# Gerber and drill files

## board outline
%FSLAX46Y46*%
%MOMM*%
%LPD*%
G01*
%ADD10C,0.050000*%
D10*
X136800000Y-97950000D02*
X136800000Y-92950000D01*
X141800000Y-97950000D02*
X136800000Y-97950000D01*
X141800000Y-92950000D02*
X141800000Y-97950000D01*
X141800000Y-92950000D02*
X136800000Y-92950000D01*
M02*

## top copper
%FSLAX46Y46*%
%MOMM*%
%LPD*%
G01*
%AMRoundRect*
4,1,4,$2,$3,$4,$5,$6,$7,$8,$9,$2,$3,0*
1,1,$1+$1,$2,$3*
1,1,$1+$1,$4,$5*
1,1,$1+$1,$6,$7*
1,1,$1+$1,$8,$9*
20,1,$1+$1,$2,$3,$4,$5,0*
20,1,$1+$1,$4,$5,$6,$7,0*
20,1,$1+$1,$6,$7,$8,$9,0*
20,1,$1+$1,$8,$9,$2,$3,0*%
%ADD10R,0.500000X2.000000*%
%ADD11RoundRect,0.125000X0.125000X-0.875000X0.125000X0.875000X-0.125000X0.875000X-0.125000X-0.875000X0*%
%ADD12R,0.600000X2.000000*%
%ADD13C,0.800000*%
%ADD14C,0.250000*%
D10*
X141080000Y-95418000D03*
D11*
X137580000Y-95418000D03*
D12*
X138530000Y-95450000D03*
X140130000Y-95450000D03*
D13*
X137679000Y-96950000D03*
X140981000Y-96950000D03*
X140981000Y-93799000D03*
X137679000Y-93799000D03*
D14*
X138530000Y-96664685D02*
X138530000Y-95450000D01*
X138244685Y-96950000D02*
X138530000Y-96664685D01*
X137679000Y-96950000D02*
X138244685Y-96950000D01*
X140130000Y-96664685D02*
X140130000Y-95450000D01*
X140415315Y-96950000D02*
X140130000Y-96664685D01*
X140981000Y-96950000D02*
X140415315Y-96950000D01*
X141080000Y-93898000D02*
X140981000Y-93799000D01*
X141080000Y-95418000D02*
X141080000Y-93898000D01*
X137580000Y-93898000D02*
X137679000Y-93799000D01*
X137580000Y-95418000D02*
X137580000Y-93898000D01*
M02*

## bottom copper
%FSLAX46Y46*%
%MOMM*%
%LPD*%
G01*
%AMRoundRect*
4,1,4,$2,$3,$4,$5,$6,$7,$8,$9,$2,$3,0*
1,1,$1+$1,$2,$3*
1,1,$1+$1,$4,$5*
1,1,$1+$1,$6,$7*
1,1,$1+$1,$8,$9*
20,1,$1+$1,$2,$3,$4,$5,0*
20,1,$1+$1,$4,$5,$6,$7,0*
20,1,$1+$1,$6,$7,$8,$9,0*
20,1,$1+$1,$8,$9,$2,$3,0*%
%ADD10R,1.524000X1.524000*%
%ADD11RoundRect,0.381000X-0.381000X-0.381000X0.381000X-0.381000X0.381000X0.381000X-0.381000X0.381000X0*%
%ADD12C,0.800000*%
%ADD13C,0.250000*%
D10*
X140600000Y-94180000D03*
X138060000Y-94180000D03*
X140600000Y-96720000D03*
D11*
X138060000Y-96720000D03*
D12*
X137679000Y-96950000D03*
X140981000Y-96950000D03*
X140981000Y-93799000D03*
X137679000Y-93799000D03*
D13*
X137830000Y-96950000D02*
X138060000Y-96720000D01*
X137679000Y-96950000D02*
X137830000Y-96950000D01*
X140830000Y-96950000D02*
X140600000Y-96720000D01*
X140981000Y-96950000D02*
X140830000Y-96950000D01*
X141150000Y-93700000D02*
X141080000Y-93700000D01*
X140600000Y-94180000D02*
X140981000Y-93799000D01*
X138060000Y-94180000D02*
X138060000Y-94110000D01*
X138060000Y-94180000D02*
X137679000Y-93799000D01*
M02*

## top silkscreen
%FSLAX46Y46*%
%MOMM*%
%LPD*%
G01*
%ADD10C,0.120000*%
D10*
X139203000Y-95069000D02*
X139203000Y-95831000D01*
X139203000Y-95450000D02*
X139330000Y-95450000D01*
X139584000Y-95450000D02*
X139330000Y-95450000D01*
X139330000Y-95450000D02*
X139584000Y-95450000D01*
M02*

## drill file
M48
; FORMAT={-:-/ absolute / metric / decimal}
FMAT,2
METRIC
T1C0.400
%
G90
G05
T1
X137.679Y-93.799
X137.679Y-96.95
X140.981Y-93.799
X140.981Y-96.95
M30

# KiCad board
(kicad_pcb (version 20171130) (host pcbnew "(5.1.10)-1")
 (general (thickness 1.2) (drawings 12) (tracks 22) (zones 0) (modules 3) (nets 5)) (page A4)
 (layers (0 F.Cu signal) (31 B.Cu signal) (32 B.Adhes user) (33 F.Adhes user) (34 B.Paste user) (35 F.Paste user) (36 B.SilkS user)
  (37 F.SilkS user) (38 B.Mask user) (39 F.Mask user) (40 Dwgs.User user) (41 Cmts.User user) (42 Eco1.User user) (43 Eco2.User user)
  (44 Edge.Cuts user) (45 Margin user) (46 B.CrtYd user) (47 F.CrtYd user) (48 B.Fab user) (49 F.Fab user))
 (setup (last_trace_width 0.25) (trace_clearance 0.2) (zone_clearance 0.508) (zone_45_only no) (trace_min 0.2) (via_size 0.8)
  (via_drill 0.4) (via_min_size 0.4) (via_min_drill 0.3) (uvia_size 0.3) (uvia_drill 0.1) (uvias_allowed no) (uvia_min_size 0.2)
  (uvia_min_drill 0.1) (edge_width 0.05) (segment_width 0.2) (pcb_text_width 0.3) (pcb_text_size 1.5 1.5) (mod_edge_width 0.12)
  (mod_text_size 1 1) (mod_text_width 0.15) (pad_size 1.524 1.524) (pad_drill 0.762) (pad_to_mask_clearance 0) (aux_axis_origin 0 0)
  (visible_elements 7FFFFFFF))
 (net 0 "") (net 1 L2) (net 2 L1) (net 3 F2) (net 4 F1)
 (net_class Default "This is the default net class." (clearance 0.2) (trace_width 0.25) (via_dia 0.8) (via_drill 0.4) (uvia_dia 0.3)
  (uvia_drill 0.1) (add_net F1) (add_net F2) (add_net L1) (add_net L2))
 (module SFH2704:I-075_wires (layer F.Cu) (at 139.33 95.418 90)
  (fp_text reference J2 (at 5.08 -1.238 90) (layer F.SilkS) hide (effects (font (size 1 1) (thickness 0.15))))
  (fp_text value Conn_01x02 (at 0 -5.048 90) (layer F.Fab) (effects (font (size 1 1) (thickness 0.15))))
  (pad 2 smd rect (at 0 1.75 90) (size 2 0.5) (layers F.Cu F.Paste F.Mask) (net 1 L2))
  (pad 1 smd roundrect (at 0 -1.75 90) (size 2 0.5) (layers F.Cu F.Paste F.Mask) (roundrect_rratio 0.25) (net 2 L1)))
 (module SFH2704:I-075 (layer B.Cu) (at 139.33 95.45)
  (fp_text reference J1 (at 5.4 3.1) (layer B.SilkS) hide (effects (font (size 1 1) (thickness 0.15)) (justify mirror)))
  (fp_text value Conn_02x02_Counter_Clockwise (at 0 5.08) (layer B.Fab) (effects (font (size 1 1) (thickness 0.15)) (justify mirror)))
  (pad 4 smd rect (at 1.27 -1.27) (size 1.524 1.524) (layers B.Cu B.Paste B.Mask) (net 1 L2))
  (pad 3 smd rect (at -1.27 -1.27) (size 1.524 1.524) (layers B.Cu B.Paste B.Mask) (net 2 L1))
  (pad 2 smd rect (at 1.27 1.27) (size 1.524 1.524) (layers B.Cu B.Paste B.Mask) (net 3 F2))
  (pad 1 smd roundrect (at -1.27 1.27) (size 1.524 1.524) (layers B.Cu B.Paste B.Mask) (roundrect_rratio 0.25) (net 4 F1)))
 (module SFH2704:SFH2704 (layer F.Cu) (at 139.33 95.45 90)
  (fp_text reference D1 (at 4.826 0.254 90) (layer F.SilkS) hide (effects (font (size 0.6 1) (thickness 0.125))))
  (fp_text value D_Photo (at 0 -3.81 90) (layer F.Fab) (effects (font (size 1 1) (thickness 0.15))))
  (pad 1 smd rect (at 0 -0.8 90) (size 2 0.6) (layers F.Cu F.Paste F.Mask) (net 4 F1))
  (pad 2 smd rect (at 0 0.8 90) (size 2 0.6) (layers F.Cu F.Paste F.Mask) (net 3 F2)))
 (gr_line (start 136.8 97.95) (end 136.8 92.95) (layer Edge.Cuts) (width 0.05))
 (gr_line (start 141.8 97.95) (end 136.8 97.95) (layer Edge.Cuts) (width 0.05))
 (gr_line (start 141.8 92.95) (end 141.8 97.95) (layer Edge.Cuts) (width 0.05))
 (gr_line (start 141.8 92.95) (end 136.8 92.95) (layer Edge.Cuts) (width 0.05))
 (gr_line (start 139.203 95.069) (end 139.203 95.831) (layer F.SilkS) (width 0.12))
 (gr_line (start 139.203 95.45) (end 139.33 95.45) (layer F.SilkS) (width 0.12))
 (gr_line (start 139.584 95.45) (end 139.33 95.45) (layer F.SilkS) (width 0.12))
 (gr_line (start 139.33 95.45) (end 139.584 95.45) (layer F.SilkS) (width 0.12))
 (via blind (at 137.679 96.95) (size 0.8) (drill 0.4) (layers F.Cu B.Cu) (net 4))
 (segment (start 137.83 96.95) (end 138.06 96.72) (width 0.25) (layer B.Cu) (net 4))
 (segment (start 137.679 96.95) (end 137.83 96.95) (width 0.25) (layer B.Cu) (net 4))
 (segment (start 138.53 96.664685) (end 138.53 95.45) (width 0.25) (layer F.Cu) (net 4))
 (segment (start 138.244685 96.95) (end 138.53 96.664685) (width 0.25) (layer F.Cu) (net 4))
 (segment (start 137.679 96.95) (end 138.244685 96.95) (width 0.25) (layer F.Cu) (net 4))
 (via blind (at 140.981 96.95) (size 0.8) (drill 0.4) (layers F.Cu B.Cu) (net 3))
 (segment (start 140.83 96.95) (end 140.6 96.72) (width 0.25) (layer B.Cu) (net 3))
 (segment (start 140.981 96.95) (end 140.83 96.95) (width 0.25) (layer B.Cu) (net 3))
 (segment (start 140.13 96.664685) (end 140.13 95.45) (width 0.25) (layer F.Cu) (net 3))
 (segment (start 140.415315 96.95) (end 140.13 96.664685) (width 0.25) (layer F.Cu) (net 3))
 (segment (start 140.981 96.95) (end 140.415315 96.95) (width 0.25) (layer F.Cu) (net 3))
 (via blind (at 140.981 93.799) (size 0.8) (drill 0.4) (layers F.Cu B.Cu) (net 1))
 (segment (start 141.15 93.7) (end 141.08 93.7) (width 0.25) (layer B.Cu) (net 1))
 (segment (start 141.08 93.898) (end 140.981 93.799) (width 0.25) (layer F.Cu) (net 1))
 (segment (start 141.08 95.418) (end 141.08 93.898) (width 0.25) (layer F.Cu) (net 1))
 (segment (start 140.6 94.18) (end 140.981 93.799) (width 0.25) (layer B.Cu) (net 1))
 (segment (start 138.06 94.18) (end 138.06 94.11) (width 0.25) (layer B.Cu) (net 2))
 (segment (start 137.58 93.898) (end 137.679 93.799) (width 0.25) (layer F.Cu) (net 2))
 (segment (start 137.58 95.418) (end 137.58 93.898) (width 0.25) (layer F.Cu) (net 2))
 (segment (start 138.06 94.18) (end 137.679 93.799) (width 0.25) (layer B.Cu) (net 2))
 (via blind (at 137.679 93.799) (size 0.8) (drill 0.4) (layers F.Cu B.Cu) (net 2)))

